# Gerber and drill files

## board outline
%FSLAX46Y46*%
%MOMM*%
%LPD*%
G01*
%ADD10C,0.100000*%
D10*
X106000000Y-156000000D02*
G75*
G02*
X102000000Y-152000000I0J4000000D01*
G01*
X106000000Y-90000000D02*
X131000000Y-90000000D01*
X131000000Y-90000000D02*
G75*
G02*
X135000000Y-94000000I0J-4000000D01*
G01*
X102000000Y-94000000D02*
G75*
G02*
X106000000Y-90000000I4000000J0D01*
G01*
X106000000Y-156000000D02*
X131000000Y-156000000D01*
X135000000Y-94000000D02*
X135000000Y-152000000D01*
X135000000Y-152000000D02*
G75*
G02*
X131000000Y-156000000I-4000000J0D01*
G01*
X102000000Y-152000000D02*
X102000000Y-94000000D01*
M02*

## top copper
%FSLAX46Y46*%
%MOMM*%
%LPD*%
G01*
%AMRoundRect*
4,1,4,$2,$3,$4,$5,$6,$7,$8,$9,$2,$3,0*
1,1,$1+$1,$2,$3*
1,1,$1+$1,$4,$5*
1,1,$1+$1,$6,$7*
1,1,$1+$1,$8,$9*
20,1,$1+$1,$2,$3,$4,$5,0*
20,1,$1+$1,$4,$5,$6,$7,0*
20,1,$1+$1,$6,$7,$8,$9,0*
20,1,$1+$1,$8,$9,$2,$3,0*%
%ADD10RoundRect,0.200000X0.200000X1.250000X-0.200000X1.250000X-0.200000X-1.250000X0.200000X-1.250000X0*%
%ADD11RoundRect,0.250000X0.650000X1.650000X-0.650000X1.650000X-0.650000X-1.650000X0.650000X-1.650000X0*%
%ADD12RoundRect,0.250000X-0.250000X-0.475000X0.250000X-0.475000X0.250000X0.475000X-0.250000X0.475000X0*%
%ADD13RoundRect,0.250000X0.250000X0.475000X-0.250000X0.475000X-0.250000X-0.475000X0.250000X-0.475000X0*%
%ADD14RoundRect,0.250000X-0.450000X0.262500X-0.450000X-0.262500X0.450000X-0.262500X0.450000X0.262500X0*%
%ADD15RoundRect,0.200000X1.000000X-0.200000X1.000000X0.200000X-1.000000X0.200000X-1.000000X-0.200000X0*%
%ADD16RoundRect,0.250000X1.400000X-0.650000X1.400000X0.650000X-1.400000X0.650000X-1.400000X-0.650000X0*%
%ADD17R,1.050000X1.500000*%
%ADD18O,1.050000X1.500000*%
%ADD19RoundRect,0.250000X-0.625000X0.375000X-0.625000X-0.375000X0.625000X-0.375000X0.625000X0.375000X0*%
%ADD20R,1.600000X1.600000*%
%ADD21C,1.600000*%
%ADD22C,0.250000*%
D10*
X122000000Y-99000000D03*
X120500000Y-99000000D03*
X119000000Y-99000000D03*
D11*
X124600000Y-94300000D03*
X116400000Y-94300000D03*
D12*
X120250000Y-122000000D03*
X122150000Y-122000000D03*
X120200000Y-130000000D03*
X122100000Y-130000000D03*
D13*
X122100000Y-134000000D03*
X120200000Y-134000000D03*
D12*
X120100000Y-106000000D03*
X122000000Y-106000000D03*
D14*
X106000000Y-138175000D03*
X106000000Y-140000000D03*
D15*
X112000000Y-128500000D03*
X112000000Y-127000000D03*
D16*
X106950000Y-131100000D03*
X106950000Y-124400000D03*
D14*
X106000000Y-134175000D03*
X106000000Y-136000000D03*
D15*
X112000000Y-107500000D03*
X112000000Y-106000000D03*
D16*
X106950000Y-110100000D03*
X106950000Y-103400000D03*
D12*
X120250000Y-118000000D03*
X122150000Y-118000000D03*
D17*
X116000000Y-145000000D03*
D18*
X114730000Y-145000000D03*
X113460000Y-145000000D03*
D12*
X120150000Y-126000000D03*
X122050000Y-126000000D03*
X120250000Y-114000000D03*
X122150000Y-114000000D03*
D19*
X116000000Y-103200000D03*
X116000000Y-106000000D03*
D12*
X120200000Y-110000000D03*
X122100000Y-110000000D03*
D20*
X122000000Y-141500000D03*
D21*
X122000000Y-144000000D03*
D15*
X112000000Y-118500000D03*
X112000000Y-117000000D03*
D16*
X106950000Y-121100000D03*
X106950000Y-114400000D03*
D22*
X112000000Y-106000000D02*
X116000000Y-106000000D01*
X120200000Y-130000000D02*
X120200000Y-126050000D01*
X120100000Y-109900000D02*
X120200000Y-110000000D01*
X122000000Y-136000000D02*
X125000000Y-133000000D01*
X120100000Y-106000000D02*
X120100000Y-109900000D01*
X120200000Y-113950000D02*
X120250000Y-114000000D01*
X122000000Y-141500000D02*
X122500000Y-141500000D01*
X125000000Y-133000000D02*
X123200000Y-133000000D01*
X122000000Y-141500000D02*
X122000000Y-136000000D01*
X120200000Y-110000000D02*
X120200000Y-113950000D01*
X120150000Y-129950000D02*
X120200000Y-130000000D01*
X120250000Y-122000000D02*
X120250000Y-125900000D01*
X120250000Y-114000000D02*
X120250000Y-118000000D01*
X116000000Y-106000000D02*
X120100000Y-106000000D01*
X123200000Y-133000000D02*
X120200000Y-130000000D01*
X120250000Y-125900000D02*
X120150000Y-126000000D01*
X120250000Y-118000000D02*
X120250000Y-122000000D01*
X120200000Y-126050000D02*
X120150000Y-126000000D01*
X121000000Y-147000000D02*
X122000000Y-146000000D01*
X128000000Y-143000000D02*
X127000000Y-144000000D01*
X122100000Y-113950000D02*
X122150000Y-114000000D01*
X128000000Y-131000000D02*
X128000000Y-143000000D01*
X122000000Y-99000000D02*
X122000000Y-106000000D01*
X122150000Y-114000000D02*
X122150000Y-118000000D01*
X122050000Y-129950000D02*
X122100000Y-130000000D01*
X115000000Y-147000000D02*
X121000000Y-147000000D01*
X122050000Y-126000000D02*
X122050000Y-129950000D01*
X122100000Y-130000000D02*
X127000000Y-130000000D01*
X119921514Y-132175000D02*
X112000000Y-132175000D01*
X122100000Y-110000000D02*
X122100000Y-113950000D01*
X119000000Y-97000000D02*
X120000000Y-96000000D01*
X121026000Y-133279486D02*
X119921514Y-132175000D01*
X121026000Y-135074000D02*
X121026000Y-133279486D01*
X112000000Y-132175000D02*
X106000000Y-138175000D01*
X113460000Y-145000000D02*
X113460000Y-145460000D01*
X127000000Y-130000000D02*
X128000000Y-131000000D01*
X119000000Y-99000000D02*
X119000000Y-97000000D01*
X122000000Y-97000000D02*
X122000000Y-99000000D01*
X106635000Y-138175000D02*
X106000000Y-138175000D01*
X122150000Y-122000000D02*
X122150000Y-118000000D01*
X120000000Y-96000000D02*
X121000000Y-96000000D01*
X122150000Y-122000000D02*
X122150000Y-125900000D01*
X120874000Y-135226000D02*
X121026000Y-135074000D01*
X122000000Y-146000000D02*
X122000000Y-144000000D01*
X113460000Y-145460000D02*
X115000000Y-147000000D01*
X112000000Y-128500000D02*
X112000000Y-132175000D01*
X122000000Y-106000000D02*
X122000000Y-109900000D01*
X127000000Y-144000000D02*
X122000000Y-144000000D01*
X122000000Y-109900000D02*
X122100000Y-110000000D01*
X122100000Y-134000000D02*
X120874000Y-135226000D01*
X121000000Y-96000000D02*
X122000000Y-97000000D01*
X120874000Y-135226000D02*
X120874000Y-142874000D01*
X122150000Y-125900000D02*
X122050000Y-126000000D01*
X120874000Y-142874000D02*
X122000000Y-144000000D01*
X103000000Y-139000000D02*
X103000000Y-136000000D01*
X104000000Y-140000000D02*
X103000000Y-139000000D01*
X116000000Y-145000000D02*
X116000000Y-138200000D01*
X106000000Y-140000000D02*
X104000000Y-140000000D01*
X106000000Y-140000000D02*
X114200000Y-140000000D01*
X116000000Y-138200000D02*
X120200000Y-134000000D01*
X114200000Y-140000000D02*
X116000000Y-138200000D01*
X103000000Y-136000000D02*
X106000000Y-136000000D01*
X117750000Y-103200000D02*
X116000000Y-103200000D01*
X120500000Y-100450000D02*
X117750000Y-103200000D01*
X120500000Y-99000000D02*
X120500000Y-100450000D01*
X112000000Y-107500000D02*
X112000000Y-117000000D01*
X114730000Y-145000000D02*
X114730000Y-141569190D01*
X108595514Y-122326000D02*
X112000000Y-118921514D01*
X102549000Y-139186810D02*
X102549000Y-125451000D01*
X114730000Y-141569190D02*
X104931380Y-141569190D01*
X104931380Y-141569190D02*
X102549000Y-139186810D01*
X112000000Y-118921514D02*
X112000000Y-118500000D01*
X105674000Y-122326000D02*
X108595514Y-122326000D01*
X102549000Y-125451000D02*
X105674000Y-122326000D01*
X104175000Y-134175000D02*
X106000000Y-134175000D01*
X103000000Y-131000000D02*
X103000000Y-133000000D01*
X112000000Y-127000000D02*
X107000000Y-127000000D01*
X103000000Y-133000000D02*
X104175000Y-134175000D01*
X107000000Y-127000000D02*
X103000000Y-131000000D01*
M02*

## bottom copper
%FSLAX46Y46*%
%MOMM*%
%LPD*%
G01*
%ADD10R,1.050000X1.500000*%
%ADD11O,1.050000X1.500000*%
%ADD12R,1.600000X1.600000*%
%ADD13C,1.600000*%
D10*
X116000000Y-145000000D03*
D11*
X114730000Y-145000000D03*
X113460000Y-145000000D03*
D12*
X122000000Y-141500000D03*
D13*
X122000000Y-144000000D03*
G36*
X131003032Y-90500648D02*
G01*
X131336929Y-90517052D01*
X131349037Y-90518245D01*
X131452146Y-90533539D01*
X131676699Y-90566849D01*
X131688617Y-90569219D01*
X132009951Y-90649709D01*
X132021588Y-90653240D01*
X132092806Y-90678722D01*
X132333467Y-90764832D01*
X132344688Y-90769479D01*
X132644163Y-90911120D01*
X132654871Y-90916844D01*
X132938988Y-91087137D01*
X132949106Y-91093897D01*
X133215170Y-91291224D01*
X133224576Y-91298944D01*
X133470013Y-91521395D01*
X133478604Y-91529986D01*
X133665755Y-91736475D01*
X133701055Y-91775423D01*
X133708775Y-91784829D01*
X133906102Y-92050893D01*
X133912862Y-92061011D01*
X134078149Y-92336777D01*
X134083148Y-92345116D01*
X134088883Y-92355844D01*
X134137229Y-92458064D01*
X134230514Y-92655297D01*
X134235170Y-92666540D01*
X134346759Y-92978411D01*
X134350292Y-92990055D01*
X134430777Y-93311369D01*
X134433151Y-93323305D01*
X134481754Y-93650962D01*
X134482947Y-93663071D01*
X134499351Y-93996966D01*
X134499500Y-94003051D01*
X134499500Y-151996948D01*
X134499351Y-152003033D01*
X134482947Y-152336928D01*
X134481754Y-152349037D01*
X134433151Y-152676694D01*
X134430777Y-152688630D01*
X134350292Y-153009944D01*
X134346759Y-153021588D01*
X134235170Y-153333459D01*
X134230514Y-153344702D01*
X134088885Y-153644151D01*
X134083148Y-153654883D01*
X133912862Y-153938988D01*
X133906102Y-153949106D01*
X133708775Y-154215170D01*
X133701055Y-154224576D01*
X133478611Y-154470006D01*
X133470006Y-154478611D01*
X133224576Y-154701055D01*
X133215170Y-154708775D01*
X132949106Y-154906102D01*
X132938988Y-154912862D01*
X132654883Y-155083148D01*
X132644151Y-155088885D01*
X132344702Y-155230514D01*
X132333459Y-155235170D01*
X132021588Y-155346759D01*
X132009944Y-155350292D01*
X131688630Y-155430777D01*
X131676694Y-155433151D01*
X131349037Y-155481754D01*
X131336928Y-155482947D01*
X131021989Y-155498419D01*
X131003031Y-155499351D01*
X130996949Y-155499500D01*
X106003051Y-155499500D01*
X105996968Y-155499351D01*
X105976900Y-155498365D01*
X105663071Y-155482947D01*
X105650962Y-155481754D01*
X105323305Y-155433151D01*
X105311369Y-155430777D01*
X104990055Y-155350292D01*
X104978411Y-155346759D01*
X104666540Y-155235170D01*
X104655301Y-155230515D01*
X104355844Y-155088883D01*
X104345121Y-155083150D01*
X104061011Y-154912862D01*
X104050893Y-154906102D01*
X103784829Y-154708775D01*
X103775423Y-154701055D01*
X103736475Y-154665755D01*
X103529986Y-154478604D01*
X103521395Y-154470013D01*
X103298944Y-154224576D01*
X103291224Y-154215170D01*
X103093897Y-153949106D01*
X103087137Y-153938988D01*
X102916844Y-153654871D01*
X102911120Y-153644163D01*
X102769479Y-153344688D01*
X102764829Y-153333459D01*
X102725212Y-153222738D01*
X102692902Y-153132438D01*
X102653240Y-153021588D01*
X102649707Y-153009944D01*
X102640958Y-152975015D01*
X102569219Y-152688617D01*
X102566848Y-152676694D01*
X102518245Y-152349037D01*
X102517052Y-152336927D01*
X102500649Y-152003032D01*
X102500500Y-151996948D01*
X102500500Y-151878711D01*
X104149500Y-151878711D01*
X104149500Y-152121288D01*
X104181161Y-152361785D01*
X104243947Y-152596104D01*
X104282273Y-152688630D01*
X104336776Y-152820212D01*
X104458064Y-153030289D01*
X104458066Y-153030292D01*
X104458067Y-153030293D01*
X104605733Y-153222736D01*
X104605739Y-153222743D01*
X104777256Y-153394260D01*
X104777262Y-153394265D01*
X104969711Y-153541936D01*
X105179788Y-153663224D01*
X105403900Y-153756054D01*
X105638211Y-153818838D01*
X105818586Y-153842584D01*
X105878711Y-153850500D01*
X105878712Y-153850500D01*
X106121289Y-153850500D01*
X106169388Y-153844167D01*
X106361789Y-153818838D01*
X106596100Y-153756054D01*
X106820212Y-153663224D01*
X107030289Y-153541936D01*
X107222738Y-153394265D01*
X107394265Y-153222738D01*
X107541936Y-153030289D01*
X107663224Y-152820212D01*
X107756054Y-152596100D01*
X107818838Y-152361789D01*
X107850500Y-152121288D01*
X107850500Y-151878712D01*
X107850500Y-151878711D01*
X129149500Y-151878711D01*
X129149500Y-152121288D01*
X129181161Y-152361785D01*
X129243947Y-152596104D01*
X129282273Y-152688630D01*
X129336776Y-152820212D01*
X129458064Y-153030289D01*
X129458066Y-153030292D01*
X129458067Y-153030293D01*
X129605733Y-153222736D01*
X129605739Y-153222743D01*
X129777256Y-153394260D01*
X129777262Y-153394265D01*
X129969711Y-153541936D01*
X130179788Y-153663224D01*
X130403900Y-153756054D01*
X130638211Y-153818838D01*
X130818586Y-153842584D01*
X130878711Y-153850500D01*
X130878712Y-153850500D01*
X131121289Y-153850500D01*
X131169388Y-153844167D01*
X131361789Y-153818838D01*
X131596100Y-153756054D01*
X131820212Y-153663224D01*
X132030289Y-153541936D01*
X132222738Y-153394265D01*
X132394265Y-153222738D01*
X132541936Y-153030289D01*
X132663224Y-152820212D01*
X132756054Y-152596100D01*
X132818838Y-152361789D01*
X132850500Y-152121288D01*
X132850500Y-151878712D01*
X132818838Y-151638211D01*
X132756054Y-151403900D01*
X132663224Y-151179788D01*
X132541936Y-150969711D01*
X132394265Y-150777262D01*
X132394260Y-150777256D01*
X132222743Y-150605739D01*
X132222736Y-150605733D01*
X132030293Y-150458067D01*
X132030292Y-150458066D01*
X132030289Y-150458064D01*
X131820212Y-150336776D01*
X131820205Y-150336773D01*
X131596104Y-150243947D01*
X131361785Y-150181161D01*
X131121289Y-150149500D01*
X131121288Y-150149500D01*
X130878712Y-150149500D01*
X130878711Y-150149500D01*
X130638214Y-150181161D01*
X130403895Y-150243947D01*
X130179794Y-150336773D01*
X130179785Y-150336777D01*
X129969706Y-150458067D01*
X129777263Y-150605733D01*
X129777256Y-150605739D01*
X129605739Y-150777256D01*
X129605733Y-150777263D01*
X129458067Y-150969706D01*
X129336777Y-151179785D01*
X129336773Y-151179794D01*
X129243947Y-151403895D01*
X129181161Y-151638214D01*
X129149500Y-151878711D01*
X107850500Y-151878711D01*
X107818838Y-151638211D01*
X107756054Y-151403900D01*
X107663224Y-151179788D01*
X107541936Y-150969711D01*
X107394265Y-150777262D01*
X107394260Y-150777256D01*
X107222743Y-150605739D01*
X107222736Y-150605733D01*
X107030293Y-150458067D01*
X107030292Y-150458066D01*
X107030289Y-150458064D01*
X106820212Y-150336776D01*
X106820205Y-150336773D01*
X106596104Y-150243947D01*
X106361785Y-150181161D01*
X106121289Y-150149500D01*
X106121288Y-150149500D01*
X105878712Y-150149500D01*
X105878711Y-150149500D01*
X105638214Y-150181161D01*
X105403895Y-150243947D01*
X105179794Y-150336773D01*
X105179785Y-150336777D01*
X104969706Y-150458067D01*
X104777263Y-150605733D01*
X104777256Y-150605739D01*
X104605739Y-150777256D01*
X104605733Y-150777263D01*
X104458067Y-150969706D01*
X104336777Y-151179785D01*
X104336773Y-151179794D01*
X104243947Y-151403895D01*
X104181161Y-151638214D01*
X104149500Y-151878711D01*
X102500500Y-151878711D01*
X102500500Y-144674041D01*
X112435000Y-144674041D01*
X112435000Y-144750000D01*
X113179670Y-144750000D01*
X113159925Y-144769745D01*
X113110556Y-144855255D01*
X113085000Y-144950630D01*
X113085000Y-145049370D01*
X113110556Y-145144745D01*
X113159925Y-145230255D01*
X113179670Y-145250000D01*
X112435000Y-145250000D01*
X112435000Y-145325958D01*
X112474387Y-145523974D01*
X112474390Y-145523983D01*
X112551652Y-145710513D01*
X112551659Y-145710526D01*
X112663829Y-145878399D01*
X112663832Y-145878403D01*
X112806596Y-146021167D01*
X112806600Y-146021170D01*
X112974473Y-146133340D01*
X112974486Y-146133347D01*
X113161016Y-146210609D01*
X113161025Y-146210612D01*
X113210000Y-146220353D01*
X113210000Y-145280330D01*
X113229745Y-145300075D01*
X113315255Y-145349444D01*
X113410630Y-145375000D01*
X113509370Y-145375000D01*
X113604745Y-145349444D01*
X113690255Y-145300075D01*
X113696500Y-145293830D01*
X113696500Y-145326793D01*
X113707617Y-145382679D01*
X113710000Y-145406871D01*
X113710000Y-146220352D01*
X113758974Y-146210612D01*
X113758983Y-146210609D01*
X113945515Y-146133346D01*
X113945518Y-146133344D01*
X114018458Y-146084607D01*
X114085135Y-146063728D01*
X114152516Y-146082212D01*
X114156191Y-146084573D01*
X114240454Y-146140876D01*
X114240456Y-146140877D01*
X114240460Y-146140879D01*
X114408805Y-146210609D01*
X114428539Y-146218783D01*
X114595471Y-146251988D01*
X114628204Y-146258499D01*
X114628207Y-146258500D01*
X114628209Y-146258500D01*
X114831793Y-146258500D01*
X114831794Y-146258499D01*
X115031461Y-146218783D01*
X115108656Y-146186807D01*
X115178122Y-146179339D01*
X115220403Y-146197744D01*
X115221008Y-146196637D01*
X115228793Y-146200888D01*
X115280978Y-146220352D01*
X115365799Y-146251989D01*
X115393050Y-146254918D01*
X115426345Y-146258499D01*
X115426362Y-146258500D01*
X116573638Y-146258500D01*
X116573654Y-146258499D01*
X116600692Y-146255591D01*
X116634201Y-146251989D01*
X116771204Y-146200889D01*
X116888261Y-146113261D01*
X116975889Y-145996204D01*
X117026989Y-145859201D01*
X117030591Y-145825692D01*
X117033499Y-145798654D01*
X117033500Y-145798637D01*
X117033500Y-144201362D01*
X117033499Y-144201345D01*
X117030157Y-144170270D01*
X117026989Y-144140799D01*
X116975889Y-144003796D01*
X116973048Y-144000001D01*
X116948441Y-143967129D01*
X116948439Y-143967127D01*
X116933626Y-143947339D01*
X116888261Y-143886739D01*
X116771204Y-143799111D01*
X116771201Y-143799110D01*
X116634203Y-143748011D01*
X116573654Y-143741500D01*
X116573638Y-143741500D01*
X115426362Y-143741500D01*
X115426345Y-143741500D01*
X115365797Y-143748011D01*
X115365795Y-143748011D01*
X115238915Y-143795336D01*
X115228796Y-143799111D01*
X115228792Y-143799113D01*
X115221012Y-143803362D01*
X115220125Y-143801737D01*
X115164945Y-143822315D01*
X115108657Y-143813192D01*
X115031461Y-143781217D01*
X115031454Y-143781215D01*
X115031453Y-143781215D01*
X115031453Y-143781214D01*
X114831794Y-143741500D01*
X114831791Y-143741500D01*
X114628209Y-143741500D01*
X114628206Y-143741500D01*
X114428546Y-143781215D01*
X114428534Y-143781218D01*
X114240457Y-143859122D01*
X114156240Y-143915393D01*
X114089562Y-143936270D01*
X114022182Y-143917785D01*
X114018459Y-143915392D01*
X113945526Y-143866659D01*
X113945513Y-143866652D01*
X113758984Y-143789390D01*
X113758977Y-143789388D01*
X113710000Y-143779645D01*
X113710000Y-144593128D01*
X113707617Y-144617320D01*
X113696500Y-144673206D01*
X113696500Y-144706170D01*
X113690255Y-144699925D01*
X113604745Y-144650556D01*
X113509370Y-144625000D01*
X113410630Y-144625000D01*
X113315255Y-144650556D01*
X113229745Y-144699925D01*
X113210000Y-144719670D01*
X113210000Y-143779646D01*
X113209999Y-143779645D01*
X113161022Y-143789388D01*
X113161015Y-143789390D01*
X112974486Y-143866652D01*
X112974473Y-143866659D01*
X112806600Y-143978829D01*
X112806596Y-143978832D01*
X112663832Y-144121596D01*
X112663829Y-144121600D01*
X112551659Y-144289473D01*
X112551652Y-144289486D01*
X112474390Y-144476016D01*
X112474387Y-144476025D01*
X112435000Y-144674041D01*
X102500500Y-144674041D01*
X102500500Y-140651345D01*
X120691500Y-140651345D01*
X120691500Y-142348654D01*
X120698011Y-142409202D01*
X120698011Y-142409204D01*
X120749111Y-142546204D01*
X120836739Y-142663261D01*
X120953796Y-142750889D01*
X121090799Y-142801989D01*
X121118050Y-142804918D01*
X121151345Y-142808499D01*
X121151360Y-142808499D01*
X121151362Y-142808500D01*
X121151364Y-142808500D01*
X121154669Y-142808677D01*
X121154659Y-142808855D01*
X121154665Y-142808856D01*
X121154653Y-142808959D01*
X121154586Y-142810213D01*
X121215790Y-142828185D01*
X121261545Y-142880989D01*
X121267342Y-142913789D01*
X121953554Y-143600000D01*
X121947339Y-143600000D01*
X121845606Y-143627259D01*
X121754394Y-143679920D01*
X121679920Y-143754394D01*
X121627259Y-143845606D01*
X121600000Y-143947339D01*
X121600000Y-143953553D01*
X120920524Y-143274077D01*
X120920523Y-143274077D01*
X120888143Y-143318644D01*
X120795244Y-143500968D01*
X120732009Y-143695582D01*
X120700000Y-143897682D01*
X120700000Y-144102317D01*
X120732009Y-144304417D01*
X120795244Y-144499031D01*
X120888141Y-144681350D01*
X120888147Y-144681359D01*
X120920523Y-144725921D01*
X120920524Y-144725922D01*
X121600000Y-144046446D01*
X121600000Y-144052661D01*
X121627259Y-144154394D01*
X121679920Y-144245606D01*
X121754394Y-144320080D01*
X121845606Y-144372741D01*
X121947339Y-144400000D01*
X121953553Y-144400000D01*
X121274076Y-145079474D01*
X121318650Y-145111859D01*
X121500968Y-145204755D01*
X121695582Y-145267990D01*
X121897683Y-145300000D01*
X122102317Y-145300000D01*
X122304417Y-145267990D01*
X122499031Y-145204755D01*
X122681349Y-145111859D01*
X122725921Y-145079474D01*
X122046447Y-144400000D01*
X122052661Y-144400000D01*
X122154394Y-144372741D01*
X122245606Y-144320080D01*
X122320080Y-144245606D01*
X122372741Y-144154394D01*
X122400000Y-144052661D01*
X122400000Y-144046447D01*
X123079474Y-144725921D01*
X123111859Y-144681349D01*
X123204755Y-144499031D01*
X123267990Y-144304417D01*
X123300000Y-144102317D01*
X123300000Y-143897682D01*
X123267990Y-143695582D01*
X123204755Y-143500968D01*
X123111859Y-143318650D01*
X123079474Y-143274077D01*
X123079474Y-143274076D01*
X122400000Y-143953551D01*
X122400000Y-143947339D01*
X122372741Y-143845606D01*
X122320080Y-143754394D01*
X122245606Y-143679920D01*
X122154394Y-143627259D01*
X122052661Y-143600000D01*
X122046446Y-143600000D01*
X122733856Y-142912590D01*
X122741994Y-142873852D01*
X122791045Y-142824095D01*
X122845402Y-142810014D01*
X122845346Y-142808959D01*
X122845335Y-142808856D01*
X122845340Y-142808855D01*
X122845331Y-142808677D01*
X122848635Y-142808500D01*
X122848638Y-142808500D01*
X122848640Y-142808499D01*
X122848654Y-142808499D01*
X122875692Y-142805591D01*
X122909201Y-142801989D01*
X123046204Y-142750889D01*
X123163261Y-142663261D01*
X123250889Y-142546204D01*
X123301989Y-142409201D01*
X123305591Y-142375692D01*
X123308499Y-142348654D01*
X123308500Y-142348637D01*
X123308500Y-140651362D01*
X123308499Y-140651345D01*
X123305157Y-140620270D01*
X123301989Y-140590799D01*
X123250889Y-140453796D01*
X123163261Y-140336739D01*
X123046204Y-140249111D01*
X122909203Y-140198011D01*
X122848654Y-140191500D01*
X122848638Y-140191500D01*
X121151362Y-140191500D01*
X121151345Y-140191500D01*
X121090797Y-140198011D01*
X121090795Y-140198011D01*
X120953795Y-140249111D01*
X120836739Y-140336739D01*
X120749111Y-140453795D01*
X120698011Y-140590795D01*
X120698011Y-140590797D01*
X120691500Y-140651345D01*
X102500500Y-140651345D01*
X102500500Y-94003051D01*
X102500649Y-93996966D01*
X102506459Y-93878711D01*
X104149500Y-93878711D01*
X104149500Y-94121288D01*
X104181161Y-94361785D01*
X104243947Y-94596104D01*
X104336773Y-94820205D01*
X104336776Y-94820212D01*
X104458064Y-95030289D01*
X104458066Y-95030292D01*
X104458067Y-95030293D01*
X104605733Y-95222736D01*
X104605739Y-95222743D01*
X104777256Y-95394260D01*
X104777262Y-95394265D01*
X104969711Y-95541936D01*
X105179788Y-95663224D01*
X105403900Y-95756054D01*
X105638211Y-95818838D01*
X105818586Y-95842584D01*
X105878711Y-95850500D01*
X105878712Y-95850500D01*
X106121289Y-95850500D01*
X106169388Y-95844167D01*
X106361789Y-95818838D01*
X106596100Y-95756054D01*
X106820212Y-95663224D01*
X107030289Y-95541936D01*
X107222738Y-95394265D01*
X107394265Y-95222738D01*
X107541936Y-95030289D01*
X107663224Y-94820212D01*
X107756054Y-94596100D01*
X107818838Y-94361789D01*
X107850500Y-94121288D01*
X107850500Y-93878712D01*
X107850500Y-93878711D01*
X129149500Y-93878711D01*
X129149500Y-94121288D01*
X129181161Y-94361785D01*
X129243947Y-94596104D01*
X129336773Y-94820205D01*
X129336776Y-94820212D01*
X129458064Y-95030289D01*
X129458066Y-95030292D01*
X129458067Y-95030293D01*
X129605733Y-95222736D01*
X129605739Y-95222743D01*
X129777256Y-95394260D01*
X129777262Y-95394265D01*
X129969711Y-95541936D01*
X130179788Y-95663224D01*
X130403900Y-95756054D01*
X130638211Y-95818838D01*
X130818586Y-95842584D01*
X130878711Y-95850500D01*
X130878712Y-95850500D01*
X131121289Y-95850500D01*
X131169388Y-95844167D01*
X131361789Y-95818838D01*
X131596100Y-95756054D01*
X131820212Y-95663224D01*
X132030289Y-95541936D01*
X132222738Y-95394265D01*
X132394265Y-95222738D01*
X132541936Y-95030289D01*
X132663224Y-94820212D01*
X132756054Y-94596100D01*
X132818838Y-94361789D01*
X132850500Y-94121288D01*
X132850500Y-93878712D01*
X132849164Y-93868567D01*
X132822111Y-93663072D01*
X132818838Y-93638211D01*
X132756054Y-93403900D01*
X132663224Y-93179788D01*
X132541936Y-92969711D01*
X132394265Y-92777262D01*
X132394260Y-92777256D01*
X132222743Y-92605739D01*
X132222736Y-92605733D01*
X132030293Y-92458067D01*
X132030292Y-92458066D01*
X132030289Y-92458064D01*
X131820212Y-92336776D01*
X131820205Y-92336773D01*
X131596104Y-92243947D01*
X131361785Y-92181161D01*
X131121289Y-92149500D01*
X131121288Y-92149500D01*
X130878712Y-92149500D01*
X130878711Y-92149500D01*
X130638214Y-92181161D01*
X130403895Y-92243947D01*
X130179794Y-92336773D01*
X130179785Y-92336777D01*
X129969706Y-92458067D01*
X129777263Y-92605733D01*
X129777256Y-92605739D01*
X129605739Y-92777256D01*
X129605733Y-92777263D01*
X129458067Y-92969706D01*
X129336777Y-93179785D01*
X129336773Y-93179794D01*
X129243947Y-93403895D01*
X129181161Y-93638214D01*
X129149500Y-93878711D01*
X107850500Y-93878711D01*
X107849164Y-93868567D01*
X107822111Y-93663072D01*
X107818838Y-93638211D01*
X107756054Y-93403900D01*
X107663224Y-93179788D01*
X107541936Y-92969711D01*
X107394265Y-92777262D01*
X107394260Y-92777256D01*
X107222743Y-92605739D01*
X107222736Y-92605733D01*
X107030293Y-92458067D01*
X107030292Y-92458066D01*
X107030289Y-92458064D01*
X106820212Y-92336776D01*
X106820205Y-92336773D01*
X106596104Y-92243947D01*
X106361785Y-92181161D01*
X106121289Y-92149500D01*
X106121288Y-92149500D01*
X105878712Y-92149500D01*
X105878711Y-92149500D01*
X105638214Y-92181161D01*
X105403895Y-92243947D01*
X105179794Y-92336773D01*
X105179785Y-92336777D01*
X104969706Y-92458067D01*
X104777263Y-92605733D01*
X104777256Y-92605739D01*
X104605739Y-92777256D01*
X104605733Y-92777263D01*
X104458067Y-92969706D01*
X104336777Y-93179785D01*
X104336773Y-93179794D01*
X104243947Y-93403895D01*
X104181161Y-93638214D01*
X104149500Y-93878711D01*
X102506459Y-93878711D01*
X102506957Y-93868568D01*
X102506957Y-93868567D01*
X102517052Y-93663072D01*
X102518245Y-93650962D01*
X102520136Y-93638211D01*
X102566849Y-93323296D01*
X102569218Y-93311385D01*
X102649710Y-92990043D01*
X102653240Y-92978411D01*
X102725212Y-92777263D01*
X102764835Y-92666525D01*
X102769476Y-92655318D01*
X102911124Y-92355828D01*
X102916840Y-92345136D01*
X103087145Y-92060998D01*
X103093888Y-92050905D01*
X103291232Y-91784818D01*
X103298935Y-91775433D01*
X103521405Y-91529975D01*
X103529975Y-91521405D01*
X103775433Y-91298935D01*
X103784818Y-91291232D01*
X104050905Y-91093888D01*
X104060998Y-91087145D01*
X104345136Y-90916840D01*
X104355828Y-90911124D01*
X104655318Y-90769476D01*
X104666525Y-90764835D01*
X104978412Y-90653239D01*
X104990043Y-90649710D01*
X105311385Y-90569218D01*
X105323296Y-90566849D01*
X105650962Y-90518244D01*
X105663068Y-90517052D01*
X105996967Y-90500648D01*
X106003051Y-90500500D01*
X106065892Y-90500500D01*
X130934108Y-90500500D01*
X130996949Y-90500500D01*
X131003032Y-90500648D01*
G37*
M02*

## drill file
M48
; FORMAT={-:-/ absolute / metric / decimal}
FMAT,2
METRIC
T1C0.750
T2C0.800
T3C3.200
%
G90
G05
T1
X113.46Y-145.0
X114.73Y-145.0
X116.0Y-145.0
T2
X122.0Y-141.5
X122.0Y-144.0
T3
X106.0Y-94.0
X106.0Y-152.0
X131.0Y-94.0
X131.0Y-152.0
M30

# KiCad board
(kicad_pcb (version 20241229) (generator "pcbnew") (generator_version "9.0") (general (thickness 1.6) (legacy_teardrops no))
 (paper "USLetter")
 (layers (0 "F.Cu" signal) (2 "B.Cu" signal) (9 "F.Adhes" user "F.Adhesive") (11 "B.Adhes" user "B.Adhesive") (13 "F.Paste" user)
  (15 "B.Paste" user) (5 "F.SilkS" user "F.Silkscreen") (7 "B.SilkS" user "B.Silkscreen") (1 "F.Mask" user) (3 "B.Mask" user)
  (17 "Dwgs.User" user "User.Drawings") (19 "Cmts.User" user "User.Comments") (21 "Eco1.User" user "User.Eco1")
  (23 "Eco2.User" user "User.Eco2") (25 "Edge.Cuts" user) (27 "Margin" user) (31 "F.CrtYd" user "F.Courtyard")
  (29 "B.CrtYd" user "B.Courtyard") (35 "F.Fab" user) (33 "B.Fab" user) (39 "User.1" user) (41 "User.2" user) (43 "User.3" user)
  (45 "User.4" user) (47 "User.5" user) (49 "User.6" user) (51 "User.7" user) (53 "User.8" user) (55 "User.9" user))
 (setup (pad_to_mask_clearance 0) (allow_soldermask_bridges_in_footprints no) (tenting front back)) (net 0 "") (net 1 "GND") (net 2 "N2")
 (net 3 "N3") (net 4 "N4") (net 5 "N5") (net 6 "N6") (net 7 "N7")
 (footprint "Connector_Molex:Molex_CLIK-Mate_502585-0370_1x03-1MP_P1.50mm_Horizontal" (layer "F.Cu") (at 120.5 96.425 180)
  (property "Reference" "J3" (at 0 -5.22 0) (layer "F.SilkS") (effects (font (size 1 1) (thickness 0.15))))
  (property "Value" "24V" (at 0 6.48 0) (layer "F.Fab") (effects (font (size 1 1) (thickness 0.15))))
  (pad "1" smd roundrect (at -1.5 -2.575 180) (size 0.8 2.9) (layers "F.Cu" "F.Mask" "F.Paste") (roundrect_rratio 0.25) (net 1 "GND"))
  (pad "2" smd roundrect (at 0 -2.575 180) (size 0.8 2.9) (layers "F.Cu" "F.Mask" "F.Paste") (roundrect_rratio 0.25) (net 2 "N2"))
  (pad "3" smd roundrect (at 1.5 -2.575 180) (size 0.8 2.9) (layers "F.Cu" "F.Mask" "F.Paste") (roundrect_rratio 0.25) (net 1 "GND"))
  (pad "MP" smd roundrect (at -4.1 2.125 180) (size 1.8 3.8) (layers "F.Cu" "F.Mask" "F.Paste") (roundrect_rratio 0.138889))
  (pad "MP" smd roundrect (at 4.1 2.125 180) (size 1.8 3.8) (layers "F.Cu" "F.Mask" "F.Paste") (roundrect_rratio 0.138889)))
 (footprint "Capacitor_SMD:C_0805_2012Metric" (layer "F.Cu") (at 121.2 122)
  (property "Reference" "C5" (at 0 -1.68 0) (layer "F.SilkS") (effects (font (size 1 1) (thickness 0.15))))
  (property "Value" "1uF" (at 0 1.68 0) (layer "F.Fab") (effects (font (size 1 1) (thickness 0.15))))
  (pad "1" smd roundrect (at -0.95 0) (size 1 1.45) (layers "F.Cu" "F.Mask" "F.Paste") (roundrect_rratio 0.25) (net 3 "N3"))
  (pad "2" smd roundrect (at 0.95 0) (size 1 1.45) (layers "F.Cu" "F.Mask" "F.Paste") (roundrect_rratio 0.25) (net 1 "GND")))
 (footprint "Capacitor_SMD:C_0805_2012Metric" (layer "F.Cu") (at 121.15 130)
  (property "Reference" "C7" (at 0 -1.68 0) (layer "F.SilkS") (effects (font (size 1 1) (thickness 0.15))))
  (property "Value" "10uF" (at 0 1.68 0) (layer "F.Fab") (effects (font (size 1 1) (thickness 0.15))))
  (pad "1" smd roundrect (at -0.95 0) (size 1 1.45) (layers "F.Cu" "F.Mask" "F.Paste") (roundrect_rratio 0.25) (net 3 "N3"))
  (pad "2" smd roundrect (at 0.95 0) (size 1 1.45) (layers "F.Cu" "F.Mask" "F.Paste") (roundrect_rratio 0.25) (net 1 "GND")))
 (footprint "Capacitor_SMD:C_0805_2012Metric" (layer "F.Cu") (at 121.15 134 180)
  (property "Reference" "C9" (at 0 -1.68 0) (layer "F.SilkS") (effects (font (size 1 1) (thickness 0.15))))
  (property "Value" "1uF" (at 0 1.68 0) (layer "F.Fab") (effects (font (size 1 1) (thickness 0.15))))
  (pad "1" smd roundrect (at -0.95 0 180) (size 1 1.45) (layers "F.Cu" "F.Mask" "F.Paste") (roundrect_rratio 0.25) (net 1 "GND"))
  (pad "2" smd roundrect (at 0.95 0 180) (size 1 1.45) (layers "F.Cu" "F.Mask" "F.Paste") (roundrect_rratio 0.25) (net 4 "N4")))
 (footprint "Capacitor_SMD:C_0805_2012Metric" (layer "F.Cu") (at 121.05 106)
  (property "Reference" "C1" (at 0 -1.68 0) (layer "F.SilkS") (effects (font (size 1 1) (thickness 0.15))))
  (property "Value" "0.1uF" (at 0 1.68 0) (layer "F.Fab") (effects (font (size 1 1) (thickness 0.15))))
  (pad "1" smd roundrect (at -0.95 0) (size 1 1.45) (layers "F.Cu" "F.Mask" "F.Paste") (roundrect_rratio 0.25) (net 3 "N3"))
  (pad "2" smd roundrect (at 0.95 0) (size 1 1.45) (layers "F.Cu" "F.Mask" "F.Paste") (roundrect_rratio 0.25) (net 1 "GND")))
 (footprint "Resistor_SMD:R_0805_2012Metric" (layer "F.Cu") (at 106 139.0875 -90)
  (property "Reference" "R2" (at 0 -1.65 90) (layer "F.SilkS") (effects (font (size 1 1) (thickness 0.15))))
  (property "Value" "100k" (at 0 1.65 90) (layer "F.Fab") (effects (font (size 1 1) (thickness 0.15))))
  (pad "1" smd roundrect (at -0.9125 0 270) (size 1.025 1.4) (layers "F.Cu" "F.Mask" "F.Paste") (roundrect_rratio 0.243902) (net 1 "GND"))
  (pad "2" smd roundrect (at 0.9125 0 270) (size 1.025 1.4) (layers "F.Cu" "F.Mask" "F.Paste") (roundrect_rratio 0.243902) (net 4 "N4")))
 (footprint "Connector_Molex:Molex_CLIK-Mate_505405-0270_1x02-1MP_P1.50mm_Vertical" (layer "F.Cu") (at 109.25 127.75 90)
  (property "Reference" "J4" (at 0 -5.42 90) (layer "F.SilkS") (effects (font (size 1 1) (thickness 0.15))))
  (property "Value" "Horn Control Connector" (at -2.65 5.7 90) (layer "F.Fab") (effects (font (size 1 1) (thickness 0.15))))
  (pad "1" smd roundrect (at -0.75 2.75 90) (size 0.8 2.4) (layers "F.Cu" "F.Mask" "F.Paste") (roundrect_rratio 0.25) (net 1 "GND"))
  (pad "2" smd roundrect (at 0.75 2.75 90) (size 0.8 2.4) (layers "F.Cu" "F.Mask" "F.Paste") (roundrect_rratio 0.25) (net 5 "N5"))
  (pad "MP" smd roundrect (at -3.35 -2.3 90) (size 1.8 3.3) (layers "F.Cu" "F.Mask" "F.Paste") (roundrect_rratio 0.138889))
  (pad "MP" smd roundrect (at 3.35 -2.3 90) (size 1.8 3.3) (layers "F.Cu" "F.Mask" "F.Paste") (roundrect_rratio 0.138889)))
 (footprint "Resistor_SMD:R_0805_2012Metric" (layer "F.Cu") (at 106 135.0875 -90)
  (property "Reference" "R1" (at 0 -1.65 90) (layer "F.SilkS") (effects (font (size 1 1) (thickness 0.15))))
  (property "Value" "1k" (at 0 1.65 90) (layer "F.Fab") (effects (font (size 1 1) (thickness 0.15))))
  (pad "1" smd roundrect (at -0.9125 0 270) (size 1.025 1.4) (layers "F.Cu" "F.Mask" "F.Paste") (roundrect_rratio 0.243902) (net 5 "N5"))
  (pad "2" smd roundrect (at 0.9125 0 270) (size 1.025 1.4) (layers "F.Cu" "F.Mask" "F.Paste") (roundrect_rratio 0.243902) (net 4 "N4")))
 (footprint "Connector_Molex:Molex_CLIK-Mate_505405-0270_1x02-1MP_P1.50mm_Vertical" (layer "F.Cu") (at 109.25 106.75 90)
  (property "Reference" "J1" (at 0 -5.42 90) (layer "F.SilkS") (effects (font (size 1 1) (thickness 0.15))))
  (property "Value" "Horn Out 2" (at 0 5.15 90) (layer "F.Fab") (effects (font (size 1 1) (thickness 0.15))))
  (pad "1" smd roundrect (at -0.75 2.75 90) (size 0.8 2.4) (layers "F.Cu" "F.Mask" "F.Paste") (roundrect_rratio 0.25) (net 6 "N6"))
  (pad "2" smd roundrect (at 0.75 2.75 90) (size 0.8 2.4) (layers "F.Cu" "F.Mask" "F.Paste") (roundrect_rratio 0.25) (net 3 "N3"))
  (pad "MP" smd roundrect (at -3.35 -2.3 90) (size 1.8 3.3) (layers "F.Cu" "F.Mask" "F.Paste") (roundrect_rratio 0.138889))
  (pad "MP" smd roundrect (at 3.35 -2.3 90) (size 1.8 3.3) (layers "F.Cu" "F.Mask" "F.Paste") (roundrect_rratio 0.138889)))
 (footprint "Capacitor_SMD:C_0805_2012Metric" (layer "F.Cu") (at 121.2 118)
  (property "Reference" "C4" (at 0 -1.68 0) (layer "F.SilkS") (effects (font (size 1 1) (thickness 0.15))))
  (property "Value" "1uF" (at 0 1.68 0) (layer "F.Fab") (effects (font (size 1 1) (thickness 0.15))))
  (pad "1" smd roundrect (at -0.95 0) (size 1 1.45) (layers "F.Cu" "F.Mask" "F.Paste") (roundrect_rratio 0.25) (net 3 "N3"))
  (pad "2" smd roundrect (at 0.95 0) (size 1 1.45) (layers "F.Cu" "F.Mask" "F.Paste") (roundrect_rratio 0.25) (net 1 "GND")))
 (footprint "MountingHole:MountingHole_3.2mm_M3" (layer "F.Cu") (at 131 152)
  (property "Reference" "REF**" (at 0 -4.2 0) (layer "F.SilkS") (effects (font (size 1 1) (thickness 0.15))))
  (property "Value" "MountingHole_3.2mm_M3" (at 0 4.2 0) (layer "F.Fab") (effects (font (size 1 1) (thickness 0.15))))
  (pad "" np_thru_hole circle (at 0 0) (size 3.2 3.2) (drill 3.2) (layers "*.Cu" "*.Mask")))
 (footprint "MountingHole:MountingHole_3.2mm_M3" (layer "F.Cu") (at 106 152)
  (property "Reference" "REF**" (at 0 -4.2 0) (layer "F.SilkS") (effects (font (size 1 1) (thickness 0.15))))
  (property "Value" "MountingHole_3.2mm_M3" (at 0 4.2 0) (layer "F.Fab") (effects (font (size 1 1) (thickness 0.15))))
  (pad "" np_thru_hole circle (at 0 0) (size 3.2 3.2) (drill 3.2) (layers "*.Cu" "*.Mask")))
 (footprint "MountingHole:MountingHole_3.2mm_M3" (layer "F.Cu") (at 131 94)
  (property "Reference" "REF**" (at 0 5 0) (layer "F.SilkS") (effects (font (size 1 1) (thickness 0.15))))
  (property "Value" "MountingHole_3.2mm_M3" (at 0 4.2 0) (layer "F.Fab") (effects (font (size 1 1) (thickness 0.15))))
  (pad "" np_thru_hole circle (at 0 0) (size 3.2 3.2) (drill 3.2) (layers "*.Cu" "*.Mask")))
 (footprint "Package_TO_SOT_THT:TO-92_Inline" (layer "F.Cu") (at 116 145 180)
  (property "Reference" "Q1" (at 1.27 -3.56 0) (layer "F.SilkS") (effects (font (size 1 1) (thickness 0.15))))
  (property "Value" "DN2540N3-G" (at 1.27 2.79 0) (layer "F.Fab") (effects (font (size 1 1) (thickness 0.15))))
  (pad "1" thru_hole rect (at 0 0 180) (size 1.05 1.5) (drill 0.75) (layers "*.Cu" "*.Mask") (remove_unused_layers no) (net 4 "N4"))
  (pad "2" thru_hole oval (at 1.27 0 180) (size 1.05 1.5) (drill 0.75) (layers "*.Cu" "*.Mask") (remove_unused_layers no) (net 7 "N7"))
  (pad "3" thru_hole oval (at 2.54 0 180) (size 1.05 1.5) (drill 0.75) (layers "*.Cu" "*.Mask") (remove_unused_layers no) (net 1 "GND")))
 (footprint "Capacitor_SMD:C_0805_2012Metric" (layer "F.Cu") (at 121.1 126)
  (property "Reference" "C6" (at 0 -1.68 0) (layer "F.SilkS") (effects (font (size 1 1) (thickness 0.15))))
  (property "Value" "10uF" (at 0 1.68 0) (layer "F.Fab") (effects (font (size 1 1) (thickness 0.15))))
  (pad "1" smd roundrect (at -0.95 0) (size 1 1.45) (layers "F.Cu" "F.Mask" "F.Paste") (roundrect_rratio 0.25) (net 3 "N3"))
  (pad "2" smd roundrect (at 0.95 0) (size 1 1.45) (layers "F.Cu" "F.Mask" "F.Paste") (roundrect_rratio 0.25) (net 1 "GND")))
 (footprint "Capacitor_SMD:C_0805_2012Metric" (layer "F.Cu") (at 121.2 114)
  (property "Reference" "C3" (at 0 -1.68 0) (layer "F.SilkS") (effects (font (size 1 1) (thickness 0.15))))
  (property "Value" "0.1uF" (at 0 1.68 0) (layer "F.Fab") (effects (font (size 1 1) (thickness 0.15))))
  (pad "1" smd roundrect (at -0.95 0) (size 1 1.45) (layers "F.Cu" "F.Mask" "F.Paste") (roundrect_rratio 0.25) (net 3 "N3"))
  (pad "2" smd roundrect (at 0.95 0) (size 1 1.45) (layers "F.Cu" "F.Mask" "F.Paste") (roundrect_rratio 0.25) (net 1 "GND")))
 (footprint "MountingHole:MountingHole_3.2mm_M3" (layer "F.Cu") (at 106 94)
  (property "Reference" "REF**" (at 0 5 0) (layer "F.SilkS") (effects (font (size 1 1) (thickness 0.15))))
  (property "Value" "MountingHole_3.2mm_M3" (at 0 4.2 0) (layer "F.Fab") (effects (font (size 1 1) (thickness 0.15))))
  (pad "" np_thru_hole circle (at 0 0) (size 3.2 3.2) (drill 3.2) (layers "*.Cu" "*.Mask")))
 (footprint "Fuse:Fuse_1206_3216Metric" (layer "F.Cu") (at 116 104.6 -90)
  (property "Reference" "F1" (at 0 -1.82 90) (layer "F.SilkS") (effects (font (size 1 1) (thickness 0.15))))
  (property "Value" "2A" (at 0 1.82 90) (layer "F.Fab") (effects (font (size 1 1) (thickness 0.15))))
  (pad "1" smd roundrect (at -1.4 0 270) (size 1.25 1.75) (layers "F.Cu" "F.Mask" "F.Paste") (roundrect_rratio 0.2) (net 2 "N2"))
  (pad "2" smd roundrect (at 1.4 0 270) (size 1.25 1.75) (layers "F.Cu" "F.Mask" "F.Paste") (roundrect_rratio 0.2) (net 3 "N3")))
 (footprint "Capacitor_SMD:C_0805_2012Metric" (layer "F.Cu") (at 121.15 110)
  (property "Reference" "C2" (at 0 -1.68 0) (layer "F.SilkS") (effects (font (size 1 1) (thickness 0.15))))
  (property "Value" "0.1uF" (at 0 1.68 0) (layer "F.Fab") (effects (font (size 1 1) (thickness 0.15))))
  (pad "1" smd roundrect (at -0.95 0) (size 1 1.45) (layers "F.Cu" "F.Mask" "F.Paste") (roundrect_rratio 0.25) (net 3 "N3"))
  (pad "2" smd roundrect (at 0.95 0) (size 1 1.45) (layers "F.Cu" "F.Mask" "F.Paste") (roundrect_rratio 0.25) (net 1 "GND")))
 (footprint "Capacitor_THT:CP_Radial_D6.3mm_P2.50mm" (layer "F.Cu") (at 122 141.5 -90)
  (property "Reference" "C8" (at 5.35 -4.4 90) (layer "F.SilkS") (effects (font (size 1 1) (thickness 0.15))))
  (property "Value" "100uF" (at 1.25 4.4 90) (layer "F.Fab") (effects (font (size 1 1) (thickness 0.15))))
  (pad "1" thru_hole rect (at 0 0 270) (size 1.6 1.6) (drill 0.8) (layers "*.Cu" "*.Mask") (remove_unused_layers no) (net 3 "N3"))
  (pad "2" thru_hole circle (at 2.5 0 270) (size 1.6 1.6) (drill 0.8) (layers "*.Cu" "*.Mask") (remove_unused_layers no) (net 1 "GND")))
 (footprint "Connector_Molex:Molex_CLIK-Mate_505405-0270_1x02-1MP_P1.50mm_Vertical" (layer "F.Cu") (at 109.25 117.75 90)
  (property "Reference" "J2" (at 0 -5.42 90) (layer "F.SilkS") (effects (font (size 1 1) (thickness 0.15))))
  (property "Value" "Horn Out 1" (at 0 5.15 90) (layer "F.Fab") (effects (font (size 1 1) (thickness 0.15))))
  (pad "1" smd roundrect (at -0.75 2.75 90) (size 0.8 2.4) (layers "F.Cu" "F.Mask" "F.Paste") (roundrect_rratio 0.25) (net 7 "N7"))
  (pad "2" smd roundrect (at 0.75 2.75 90) (size 0.8 2.4) (layers "F.Cu" "F.Mask" "F.Paste") (roundrect_rratio 0.25) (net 6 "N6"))
  (pad "MP" smd roundrect (at -3.35 -2.3 90) (size 1.8 3.3) (layers "F.Cu" "F.Mask" "F.Paste") (roundrect_rratio 0.138889))
  (pad "MP" smd roundrect (at 3.35 -2.3 90) (size 1.8 3.3) (layers "F.Cu" "F.Mask" "F.Paste") (roundrect_rratio 0.138889)))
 (gr_arc (start 106 156) (mid 103.171573 154.828427) (end 102 152) (stroke (width 0.1) (type default)) (layer "Edge.Cuts"))
 (gr_line (start 106 90) (end 131 90) (stroke (width 0.1) (type default)) (layer "Edge.Cuts"))
 (gr_arc (start 131 90) (mid 133.828427 91.171573) (end 135 94) (stroke (width 0.1) (type default)) (layer "Edge.Cuts"))
 (gr_arc (start 102 94) (mid 103.171573 91.171573) (end 106 90) (stroke (width 0.1) (type default)) (layer "Edge.Cuts"))
 (gr_line (start 106 156) (end 131 156) (stroke (width 0.1) (type default)) (layer "Edge.Cuts"))
 (gr_line (start 135 94) (end 135 152) (stroke (width 0.1) (type default)) (layer "Edge.Cuts"))
 (gr_arc (start 135 152) (mid 133.828427 154.828427) (end 131 156) (stroke (width 0.1) (type default)) (layer "Edge.Cuts"))
 (gr_line (start 102 152) (end 102 94) (stroke (width 0.1) (type default)) (layer "Edge.Cuts"))
 (segment (start 112 106) (end 116 106) (width 0.25) (layer "F.Cu") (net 3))
 (segment (start 120.2 130) (end 120.2 126.05) (width 0.25) (layer "F.Cu") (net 3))
 (segment (start 120.1 109.9) (end 120.2 110) (width 0.25) (layer "F.Cu") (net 3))
 (segment (start 122 136) (end 125 133) (width 0.25) (layer "F.Cu") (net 3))
 (segment (start 120.1 106) (end 120.1 109.9) (width 0.25) (layer "F.Cu") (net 3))
 (segment (start 120.2 113.95) (end 120.25 114) (width 0.25) (layer "F.Cu") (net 3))
 (segment (start 122 141.5) (end 122.5 141.5) (width 0.25) (layer "F.Cu") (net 3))
 (segment (start 125 133) (end 123.2 133) (width 0.25) (layer "F.Cu") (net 3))
 (segment (start 122 141.5) (end 122 136) (width 0.25) (layer "F.Cu") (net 3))
 (segment (start 120.2 110) (end 120.2 113.95) (width 0.25) (layer "F.Cu") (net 3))
 (segment (start 120.15 129.95) (end 120.2 130) (width 0.25) (layer "F.Cu") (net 3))
 (segment (start 120.25 122) (end 120.25 125.9) (width 0.25) (layer "F.Cu") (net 3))
 (segment (start 120.25 114) (end 120.25 118) (width 0.25) (layer "F.Cu") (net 3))
 (segment (start 116 106) (end 120.1 106) (width 0.25) (layer "F.Cu") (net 3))
 (segment (start 123.2 133) (end 120.2 130) (width 0.25) (layer "F.Cu") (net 3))
 (segment (start 120.25 125.9) (end 120.15 126) (width 0.25) (layer "F.Cu") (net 3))
 (segment (start 120.25 118) (end 120.25 122) (width 0.25) (layer "F.Cu") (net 3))
 (segment (start 120.2 126.05) (end 120.15 126) (width 0.25) (layer "F.Cu") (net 3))
 (segment (start 121 147) (end 122 146) (width 0.25) (layer "F.Cu") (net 1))
 (segment (start 128 143) (end 127 144) (width 0.25) (layer "F.Cu") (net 1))
 (segment (start 122.1 113.95) (end 122.15 114) (width 0.25) (layer "F.Cu") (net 1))
 (segment (start 128 131) (end 128 143) (width 0.25) (layer "F.Cu") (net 1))
 (segment (start 122 99) (end 122 106) (width 0.25) (layer "F.Cu") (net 1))
 (segment (start 122.15 114) (end 122.15 118) (width 0.25) (layer "F.Cu") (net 1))
 (segment (start 122.05 129.95) (end 122.1 130) (width 0.25) (layer "F.Cu") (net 1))
 (segment (start 115 147) (end 121 147) (width 0.25) (layer "F.Cu") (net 1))
 (segment (start 122.05 126) (end 122.05 129.95) (width 0.25) (layer "F.Cu") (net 1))
 (segment (start 122.1 130) (end 127 130) (width 0.25) (layer "F.Cu") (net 1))
 (segment (start 119.921514 132.175) (end 112 132.175) (width 0.25) (layer "F.Cu") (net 1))
 (segment (start 122.1 110) (end 122.1 113.95) (width 0.25) (layer "F.Cu") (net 1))
 (segment (start 119 97) (end 120 96) (width 0.25) (layer "F.Cu") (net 1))
 (segment (start 121.026 133.279486) (end 119.921514 132.175) (width 0.25) (layer "F.Cu") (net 1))
 (segment (start 121.026 135.074) (end 121.026 133.279486) (width 0.25) (layer "F.Cu") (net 1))
 (segment (start 112 132.175) (end 106 138.175) (width 0.25) (layer "F.Cu") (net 1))
 (segment (start 113.46 145) (end 113.46 145.46) (width 0.25) (layer "F.Cu") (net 1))
 (segment (start 127 130) (end 128 131) (width 0.25) (layer "F.Cu") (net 1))
 (segment (start 119 99) (end 119 97) (width 0.25) (layer "F.Cu") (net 1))
 (segment (start 122 97) (end 122 99) (width 0.25) (layer "F.Cu") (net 1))
 (segment (start 106.635 138.175) (end 106 138.175) (width 0.25) (layer "F.Cu") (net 1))
 (segment (start 122.15 122) (end 122.15 118) (width 0.25) (layer "F.Cu") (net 1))
 (segment (start 120 96) (end 121 96) (width 0.25) (layer "F.Cu") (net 1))
 (segment (start 122.15 122) (end 122.15 125.9) (width 0.25) (layer "F.Cu") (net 1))
 (segment (start 120.874 135.226) (end 121.026 135.074) (width 0.25) (layer "F.Cu") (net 1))
 (segment (start 122 146) (end 122 144) (width 0.25) (layer "F.Cu") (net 1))
 (segment (start 113.46 145.46) (end 115 147) (width 0.25) (layer "F.Cu") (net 1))
 (segment (start 112 128.5) (end 112 132.175) (width 0.25) (layer "F.Cu") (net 1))
 (segment (start 122 106) (end 122 109.9) (width 0.25) (layer "F.Cu") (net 1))
 (segment (start 127 144) (end 122 144) (width 0.25) (layer "F.Cu") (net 1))
 (segment (start 122 109.9) (end 122.1 110) (width 0.25) (layer "F.Cu") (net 1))
 (segment (start 122.1 134) (end 120.874 135.226) (width 0.25) (layer "F.Cu") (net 1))
 (segment (start 121 96) (end 122 97) (width 0.25) (layer "F.Cu") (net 1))
 (segment (start 120.874 135.226) (end 120.874 142.874) (width 0.25) (layer "F.Cu") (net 1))
 (segment (start 122.15 125.9) (end 122.05 126) (width 0.25) (layer "F.Cu") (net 1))
 (segment (start 120.874 142.874) (end 122 144) (width 0.25) (layer "F.Cu") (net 1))
 (segment (start 103 139) (end 103 136) (width 0.25) (layer "F.Cu") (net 4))
 (segment (start 104 140) (end 103 139) (width 0.25) (layer "F.Cu") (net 4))
 (segment (start 116 145) (end 116 138.2) (width 0.25) (layer "F.Cu") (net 4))
 (segment (start 106 140) (end 104 140) (width 0.25) (layer "F.Cu") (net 4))
 (segment (start 106 140) (end 114.2 140) (width 0.25) (layer "F.Cu") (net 4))
 (segment (start 116 138.2) (end 120.2 134) (width 0.25) (layer "F.Cu") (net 4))
 (segment (start 114.2 140) (end 116 138.2) (width 0.25) (layer "F.Cu") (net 4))
 (segment (start 103 136) (end 106 136) (width 0.25) (layer "F.Cu") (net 4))
 (segment (start 117.75 103.2) (end 116 103.2) (width 0.25) (layer "F.Cu") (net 2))
 (segment (start 120.5 100.45) (end 117.75 103.2) (width 0.25) (layer "F.Cu") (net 2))
 (segment (start 120.5 99) (end 120.5 100.45) (width 0.25) (layer "F.Cu") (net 2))
 (segment (start 112 107.5) (end 112 117) (width 0.25) (layer "F.Cu") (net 6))
 (segment (start 114.73 145) (end 114.73 141.56919) (width 0.25) (layer "F.Cu") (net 7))
 (segment (start 108.595514 122.326) (end 112 118.921514) (width 0.25) (layer "F.Cu") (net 7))
 (segment (start 102.549 139.18681) (end 102.549 125.451) (width 0.25) (layer "F.Cu") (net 7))
 (segment (start 114.73 141.56919) (end 104.93138 141.56919) (width 0.25) (layer "F.Cu") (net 7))
 (segment (start 104.93138 141.56919) (end 102.549 139.18681) (width 0.25) (layer "F.Cu") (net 7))
 (segment (start 112 118.921514) (end 112 118.5) (width 0.25) (layer "F.Cu") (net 7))
 (segment (start 105.674 122.326) (end 108.595514 122.326) (width 0.25) (layer "F.Cu") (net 7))
 (segment (start 102.549 125.451) (end 105.674 122.326) (width 0.25) (layer "F.Cu") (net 7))
 (segment (start 104.175 134.175) (end 106 134.175) (width 0.25) (layer "F.Cu") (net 5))
 (segment (start 103 131) (end 103 133) (width 0.25) (layer "F.Cu") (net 5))
 (segment (start 112 127) (end 107 127) (width 0.25) (layer "F.Cu") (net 5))
 (segment (start 103 133) (end 104.175 134.175) (width 0.25) (layer "F.Cu") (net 5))
 (segment (start 107 127) (end 103 131) (width 0.25) (layer "F.Cu") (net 5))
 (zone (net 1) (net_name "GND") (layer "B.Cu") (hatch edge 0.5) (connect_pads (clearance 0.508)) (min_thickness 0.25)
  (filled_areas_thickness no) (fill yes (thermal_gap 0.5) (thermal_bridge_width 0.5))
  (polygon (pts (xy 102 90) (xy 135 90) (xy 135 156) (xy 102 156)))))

